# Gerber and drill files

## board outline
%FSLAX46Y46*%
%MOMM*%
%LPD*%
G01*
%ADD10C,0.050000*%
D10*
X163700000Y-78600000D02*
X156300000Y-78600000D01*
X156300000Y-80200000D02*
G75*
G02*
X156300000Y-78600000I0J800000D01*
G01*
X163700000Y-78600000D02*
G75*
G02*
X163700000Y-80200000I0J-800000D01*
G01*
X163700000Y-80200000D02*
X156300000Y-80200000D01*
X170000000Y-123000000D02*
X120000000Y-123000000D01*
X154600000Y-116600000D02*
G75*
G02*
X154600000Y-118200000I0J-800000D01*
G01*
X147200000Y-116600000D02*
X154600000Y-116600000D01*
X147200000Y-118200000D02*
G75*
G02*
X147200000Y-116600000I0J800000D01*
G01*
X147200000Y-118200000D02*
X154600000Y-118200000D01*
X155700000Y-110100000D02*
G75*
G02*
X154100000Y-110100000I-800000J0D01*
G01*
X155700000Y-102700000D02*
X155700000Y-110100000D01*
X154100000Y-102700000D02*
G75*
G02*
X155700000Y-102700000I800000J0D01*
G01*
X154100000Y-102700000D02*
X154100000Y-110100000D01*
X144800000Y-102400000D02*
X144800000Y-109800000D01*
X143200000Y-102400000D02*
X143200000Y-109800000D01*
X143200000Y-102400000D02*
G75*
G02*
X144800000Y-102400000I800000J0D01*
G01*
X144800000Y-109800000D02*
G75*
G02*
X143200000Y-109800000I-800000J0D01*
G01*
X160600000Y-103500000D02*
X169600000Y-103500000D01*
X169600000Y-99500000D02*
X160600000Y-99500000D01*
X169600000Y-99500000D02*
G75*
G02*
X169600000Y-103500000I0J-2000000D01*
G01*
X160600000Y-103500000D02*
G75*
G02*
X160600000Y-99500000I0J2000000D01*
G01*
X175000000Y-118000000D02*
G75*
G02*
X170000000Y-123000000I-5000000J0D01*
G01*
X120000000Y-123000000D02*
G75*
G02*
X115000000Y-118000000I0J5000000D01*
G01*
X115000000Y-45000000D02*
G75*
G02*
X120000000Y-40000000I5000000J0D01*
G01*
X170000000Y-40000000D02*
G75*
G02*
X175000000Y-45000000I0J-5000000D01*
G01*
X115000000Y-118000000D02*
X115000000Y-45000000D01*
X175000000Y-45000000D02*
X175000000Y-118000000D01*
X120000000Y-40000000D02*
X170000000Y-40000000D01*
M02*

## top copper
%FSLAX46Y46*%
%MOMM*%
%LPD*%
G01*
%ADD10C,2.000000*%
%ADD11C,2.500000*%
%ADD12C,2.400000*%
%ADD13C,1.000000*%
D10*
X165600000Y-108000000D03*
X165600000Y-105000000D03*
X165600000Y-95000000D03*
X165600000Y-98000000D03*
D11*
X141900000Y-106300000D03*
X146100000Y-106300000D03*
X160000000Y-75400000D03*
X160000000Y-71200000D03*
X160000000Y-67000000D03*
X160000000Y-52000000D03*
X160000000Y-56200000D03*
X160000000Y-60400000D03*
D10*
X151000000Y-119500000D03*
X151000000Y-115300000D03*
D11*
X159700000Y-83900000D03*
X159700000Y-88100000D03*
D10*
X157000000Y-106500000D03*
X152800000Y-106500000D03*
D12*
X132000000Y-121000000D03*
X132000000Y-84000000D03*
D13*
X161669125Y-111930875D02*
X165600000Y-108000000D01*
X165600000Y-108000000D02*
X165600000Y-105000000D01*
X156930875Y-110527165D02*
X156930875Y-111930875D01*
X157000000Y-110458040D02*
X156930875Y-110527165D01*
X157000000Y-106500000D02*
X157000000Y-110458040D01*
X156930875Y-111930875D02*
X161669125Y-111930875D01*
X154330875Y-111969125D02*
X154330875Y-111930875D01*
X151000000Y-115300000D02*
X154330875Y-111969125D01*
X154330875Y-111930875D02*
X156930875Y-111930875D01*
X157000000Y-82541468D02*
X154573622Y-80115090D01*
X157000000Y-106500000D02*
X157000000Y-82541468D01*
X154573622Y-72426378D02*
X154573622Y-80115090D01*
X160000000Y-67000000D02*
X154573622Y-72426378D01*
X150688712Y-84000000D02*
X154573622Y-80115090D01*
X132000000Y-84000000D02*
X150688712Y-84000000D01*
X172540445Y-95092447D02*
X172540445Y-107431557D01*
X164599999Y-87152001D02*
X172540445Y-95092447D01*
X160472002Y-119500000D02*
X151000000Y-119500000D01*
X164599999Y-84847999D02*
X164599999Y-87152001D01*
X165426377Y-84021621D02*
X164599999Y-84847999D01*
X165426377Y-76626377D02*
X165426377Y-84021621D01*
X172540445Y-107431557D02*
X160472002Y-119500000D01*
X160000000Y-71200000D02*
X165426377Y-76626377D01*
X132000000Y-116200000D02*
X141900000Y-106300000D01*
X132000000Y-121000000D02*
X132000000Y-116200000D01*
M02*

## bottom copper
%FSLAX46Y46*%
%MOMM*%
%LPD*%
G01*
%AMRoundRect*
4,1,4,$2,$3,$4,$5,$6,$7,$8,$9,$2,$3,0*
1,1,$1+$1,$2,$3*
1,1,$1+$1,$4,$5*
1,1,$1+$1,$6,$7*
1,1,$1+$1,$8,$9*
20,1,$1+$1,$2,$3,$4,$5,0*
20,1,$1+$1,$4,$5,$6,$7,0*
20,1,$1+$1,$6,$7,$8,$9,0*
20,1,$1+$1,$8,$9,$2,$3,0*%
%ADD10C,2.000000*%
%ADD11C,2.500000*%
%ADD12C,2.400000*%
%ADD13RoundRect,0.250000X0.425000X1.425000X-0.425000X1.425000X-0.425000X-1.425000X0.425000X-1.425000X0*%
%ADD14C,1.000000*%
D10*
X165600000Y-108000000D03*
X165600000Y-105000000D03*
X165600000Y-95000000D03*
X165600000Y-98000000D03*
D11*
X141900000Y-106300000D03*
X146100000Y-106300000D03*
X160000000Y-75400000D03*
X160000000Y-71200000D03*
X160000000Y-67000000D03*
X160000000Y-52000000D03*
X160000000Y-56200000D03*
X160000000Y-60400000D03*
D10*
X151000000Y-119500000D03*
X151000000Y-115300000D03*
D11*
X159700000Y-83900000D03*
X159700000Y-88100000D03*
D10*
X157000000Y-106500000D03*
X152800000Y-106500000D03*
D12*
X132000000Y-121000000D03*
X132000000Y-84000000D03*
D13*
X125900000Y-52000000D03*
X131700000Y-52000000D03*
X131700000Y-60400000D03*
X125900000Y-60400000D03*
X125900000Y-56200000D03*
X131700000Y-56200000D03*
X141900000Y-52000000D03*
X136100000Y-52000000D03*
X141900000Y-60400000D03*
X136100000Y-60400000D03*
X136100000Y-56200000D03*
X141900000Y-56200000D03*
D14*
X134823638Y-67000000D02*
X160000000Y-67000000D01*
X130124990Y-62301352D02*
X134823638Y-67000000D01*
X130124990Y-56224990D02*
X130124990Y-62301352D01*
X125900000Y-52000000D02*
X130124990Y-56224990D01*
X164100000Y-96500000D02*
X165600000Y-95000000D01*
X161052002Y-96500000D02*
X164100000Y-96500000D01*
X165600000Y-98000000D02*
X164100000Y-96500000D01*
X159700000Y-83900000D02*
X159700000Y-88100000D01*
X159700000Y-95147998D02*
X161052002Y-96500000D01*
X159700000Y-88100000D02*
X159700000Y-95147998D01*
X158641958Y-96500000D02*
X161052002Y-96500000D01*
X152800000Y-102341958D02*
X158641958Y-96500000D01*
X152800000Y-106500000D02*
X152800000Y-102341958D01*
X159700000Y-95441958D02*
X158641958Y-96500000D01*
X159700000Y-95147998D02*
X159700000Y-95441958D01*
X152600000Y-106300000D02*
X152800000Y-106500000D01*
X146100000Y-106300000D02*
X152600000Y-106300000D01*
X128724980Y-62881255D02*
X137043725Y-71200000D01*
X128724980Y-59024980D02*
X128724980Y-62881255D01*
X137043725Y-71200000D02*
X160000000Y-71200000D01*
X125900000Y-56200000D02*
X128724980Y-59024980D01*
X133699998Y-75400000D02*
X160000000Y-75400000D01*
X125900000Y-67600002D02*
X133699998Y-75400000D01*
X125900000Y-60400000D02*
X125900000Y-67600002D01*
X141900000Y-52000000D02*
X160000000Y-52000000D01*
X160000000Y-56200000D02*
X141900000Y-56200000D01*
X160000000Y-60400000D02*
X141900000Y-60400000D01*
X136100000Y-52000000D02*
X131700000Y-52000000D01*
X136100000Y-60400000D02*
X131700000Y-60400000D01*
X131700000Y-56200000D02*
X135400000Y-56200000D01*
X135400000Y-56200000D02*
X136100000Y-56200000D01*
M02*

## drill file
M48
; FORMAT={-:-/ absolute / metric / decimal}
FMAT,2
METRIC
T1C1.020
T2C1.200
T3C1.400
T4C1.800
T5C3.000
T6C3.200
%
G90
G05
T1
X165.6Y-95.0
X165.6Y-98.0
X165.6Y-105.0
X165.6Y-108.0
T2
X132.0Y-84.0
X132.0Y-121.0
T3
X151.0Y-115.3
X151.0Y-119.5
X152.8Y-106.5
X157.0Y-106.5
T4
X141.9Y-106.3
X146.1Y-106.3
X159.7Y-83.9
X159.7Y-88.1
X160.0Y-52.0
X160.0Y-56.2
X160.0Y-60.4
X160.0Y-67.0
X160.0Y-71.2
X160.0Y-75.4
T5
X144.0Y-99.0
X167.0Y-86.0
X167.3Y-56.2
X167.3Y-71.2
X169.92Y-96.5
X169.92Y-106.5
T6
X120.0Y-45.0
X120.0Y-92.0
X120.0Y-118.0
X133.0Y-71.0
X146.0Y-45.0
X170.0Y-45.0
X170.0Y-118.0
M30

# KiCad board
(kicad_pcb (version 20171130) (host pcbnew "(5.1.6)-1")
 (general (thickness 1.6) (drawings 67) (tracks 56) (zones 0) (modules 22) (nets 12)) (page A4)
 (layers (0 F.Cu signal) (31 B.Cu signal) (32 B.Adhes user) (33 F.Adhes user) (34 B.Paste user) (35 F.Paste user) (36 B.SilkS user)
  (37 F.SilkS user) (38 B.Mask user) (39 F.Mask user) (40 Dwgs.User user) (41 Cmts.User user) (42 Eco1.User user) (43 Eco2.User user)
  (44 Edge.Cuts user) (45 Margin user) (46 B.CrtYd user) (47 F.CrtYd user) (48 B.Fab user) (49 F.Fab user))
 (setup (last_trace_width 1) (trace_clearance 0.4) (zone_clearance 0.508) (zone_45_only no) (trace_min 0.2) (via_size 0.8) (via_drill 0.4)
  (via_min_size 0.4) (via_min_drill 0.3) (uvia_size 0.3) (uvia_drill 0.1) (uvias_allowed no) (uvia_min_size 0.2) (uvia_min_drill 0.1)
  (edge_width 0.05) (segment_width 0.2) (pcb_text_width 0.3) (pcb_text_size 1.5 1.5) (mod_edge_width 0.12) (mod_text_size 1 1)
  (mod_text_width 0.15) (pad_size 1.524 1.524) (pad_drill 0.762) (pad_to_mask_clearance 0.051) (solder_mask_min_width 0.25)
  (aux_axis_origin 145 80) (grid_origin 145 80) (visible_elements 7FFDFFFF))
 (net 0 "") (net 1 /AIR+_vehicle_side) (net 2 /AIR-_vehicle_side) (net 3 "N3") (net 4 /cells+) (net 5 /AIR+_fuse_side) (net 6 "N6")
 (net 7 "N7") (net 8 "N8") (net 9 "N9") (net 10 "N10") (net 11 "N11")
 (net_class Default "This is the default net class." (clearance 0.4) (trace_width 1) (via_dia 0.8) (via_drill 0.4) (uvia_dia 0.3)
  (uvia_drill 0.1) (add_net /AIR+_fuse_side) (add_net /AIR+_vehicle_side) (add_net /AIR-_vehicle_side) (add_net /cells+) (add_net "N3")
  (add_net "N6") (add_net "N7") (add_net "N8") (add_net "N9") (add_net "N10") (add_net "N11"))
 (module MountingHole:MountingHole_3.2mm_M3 (layer B.Cu) (at 120 92)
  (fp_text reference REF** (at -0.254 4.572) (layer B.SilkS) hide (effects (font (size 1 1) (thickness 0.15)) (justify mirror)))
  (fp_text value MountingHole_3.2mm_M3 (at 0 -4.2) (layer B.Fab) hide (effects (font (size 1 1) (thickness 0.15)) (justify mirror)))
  (pad 1 np_thru_hole circle (at 0 0) (size 3.2 3.2) (drill 3.2) (layers *.Cu *.Mask)))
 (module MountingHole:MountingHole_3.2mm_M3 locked (layer B.Cu) (at 133 71)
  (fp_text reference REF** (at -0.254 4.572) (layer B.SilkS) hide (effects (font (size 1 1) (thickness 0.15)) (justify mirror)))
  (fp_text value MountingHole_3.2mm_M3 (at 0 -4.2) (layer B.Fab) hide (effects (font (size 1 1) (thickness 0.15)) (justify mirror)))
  (pad 1 np_thru_hole circle (at 0 0) (size 3.2 3.2) (drill 3.2) (layers *.Cu *.Mask)))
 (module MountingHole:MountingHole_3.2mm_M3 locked (layer B.Cu) (at 146 45)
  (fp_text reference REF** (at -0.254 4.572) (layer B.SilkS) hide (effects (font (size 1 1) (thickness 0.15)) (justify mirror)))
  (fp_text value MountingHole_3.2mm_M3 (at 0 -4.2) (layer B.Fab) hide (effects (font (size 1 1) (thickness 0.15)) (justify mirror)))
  (pad 1 np_thru_hole circle (at 0 0) (size 3.2 3.2) (drill 3.2) (layers *.Cu *.Mask)))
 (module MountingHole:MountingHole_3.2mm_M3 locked (layer B.Cu) (at 170 45 180)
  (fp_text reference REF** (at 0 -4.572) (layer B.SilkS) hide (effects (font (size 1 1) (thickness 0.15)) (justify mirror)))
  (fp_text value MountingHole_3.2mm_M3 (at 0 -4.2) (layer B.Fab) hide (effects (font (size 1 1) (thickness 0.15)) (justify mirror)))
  (pad 1 np_thru_hole circle (at 0 0 180) (size 3.2 3.2) (drill 3.2) (layers *.Cu *.Mask)))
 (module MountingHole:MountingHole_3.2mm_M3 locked (layer B.Cu) (at 120 118)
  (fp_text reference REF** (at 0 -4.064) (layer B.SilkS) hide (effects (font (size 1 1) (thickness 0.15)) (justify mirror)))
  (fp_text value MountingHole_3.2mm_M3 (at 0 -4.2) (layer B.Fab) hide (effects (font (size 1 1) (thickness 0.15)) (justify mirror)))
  (pad 1 np_thru_hole circle (at 0 0) (size 3.2 3.2) (drill 3.2) (layers *.Cu *.Mask)))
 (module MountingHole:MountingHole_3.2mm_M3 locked (layer B.Cu) (at 170 118 180)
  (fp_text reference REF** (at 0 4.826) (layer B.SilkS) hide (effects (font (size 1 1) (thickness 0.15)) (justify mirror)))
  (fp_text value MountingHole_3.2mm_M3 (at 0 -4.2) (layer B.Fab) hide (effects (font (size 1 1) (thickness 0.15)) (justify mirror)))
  (pad 1 np_thru_hole circle (at 0 0 180) (size 3.2 3.2) (drill 3.2) (layers *.Cu *.Mask)))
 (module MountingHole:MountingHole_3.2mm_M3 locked (layer B.Cu) (at 120 45)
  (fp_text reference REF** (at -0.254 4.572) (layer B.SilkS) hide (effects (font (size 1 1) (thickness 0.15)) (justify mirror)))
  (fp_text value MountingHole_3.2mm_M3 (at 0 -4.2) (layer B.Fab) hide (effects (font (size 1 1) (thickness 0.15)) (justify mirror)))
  (pad 1 np_thru_hole circle (at 0 0) (size 3.2 3.2) (drill 3.2) (layers *.Cu *.Mask)))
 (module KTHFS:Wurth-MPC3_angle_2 (layer F.Cu) (at 165.6 105 90)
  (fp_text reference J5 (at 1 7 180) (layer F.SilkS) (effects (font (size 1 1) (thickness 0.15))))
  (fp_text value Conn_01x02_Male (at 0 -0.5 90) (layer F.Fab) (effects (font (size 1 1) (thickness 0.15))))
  (pad "" np_thru_hole circle (at -1.5 4.32 90) (size 3 3) (drill 3) (layers *.Cu *.Mask))
  (pad 2 thru_hole circle (at -3 0 90) (size 2 2) (drill 1.02) (layers *.Cu *.Mask) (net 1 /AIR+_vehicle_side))
  (pad 1 thru_hole circle (at 0 0 90) (size 2 2) (drill 1.02) (layers *.Cu *.Mask) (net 1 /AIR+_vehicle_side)))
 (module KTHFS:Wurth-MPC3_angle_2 (layer F.Cu) (at 165.6 95 90)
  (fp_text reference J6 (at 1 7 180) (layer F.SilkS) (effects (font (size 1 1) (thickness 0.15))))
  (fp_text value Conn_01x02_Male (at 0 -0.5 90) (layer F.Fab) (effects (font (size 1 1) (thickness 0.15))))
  (pad 1 thru_hole circle (at 0 0 90) (size 2 2) (drill 1.02) (layers *.Cu *.Mask) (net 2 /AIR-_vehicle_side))
  (pad 2 thru_hole circle (at -3 0 90) (size 2 2) (drill 1.02) (layers *.Cu *.Mask) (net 2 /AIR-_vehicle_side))
  (pad "" np_thru_hole circle (at -1.5 4.32 90) (size 3 3) (drill 3) (layers *.Cu *.Mask)))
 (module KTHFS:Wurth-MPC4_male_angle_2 (layer F.Cu) (at 144 99 180)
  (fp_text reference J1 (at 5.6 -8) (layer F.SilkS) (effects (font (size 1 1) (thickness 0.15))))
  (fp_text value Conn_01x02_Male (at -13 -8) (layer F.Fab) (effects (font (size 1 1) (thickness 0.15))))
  (pad "" np_thru_hole circle (at 0 0 180) (size 3 3) (drill 3) (layers *.Cu *.Mask))
  (pad 1 thru_hole circle (at 2.1 -7.3 180) (size 2.5 2.5) (drill 1.8) (layers *.Cu *.Mask) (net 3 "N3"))
  (pad 2 thru_hole circle (at -2.1 -7.3 180) (size 2.5 2.5) (drill 1.8) (layers *.Cu *.Mask) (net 2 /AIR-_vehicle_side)))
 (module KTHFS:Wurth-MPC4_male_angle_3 (layer F.Cu) (at 160 67 90)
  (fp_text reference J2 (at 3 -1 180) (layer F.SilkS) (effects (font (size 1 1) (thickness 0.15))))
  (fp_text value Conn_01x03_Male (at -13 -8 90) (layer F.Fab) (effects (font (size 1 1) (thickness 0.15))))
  (pad 3 thru_hole circle (at -8.4 0 90) (size 2.5 2.5) (drill 1.8) (layers *.Cu *.Mask) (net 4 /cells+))
  (pad 2 thru_hole circle (at -4.2 0 90) (size 2.5 2.5) (drill 1.8) (layers *.Cu *.Mask) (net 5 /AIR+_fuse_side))
  (pad 1 thru_hole circle (at 0 0 90) (size 2.5 2.5) (drill 1.8) (layers *.Cu *.Mask) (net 1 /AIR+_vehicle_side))
  (pad "" np_thru_hole circle (at -4.2 7.3 90) (size 3 3) (drill 3) (layers *.Cu *.Mask)))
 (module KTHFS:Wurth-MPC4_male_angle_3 (layer F.Cu) (at 160 52 90)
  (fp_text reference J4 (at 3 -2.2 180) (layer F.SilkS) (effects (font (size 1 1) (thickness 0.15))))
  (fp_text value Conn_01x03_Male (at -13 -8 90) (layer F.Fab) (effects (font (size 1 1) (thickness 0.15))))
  (pad "" np_thru_hole circle (at -4.2 7.3 90) (size 3 3) (drill 3) (layers *.Cu *.Mask))
  (pad 1 thru_hole circle (at 0 0 90) (size 2.5 2.5) (drill 1.8) (layers *.Cu *.Mask) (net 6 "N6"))
  (pad 2 thru_hole circle (at -4.2 0 90) (size 2.5 2.5) (drill 1.8) (layers *.Cu *.Mask) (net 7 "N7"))
  (pad 3 thru_hole circle (at -8.4 0 90) (size 2.5 2.5) (drill 1.8) (layers *.Cu *.Mask) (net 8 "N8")))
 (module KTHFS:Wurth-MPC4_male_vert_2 (layer F.Cu) (at 151 119.5 90)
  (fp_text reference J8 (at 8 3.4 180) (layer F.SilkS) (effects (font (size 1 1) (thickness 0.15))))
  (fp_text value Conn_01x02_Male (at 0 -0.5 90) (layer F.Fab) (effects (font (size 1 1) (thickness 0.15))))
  (pad 1 thru_hole circle (at 0 0 90) (size 2 2) (drill 1.4) (layers *.Cu *.Mask) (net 5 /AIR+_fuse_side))
  (pad 2 thru_hole circle (at 4.2 0 90) (size 2 2) (drill 1.4) (layers *.Cu *.Mask) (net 1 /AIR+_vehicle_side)))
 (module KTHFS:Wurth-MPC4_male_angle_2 (layer F.Cu) (at 167 86 90)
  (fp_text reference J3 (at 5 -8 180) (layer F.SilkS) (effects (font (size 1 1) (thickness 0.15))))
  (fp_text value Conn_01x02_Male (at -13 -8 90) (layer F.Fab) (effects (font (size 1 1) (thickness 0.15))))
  (pad "" np_thru_hole circle (at 0 0 90) (size 3 3) (drill 3) (layers *.Cu *.Mask))
  (pad 1 thru_hole circle (at 2.1 -7.3 90) (size 2.5 2.5) (drill 1.8) (layers *.Cu *.Mask) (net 2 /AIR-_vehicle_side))
  (pad 2 thru_hole circle (at -2.1 -7.3 90) (size 2.5 2.5) (drill 1.8) (layers *.Cu *.Mask) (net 2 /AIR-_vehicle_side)))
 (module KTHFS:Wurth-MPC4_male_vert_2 (layer F.Cu) (at 157 106.5 180)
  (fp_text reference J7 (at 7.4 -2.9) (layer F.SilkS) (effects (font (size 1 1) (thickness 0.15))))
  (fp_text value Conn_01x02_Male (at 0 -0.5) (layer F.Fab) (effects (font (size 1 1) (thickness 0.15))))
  (pad 1 thru_hole circle (at 0 0 180) (size 2 2) (drill 1.4) (layers *.Cu *.Mask) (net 1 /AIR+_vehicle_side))
  (pad 2 thru_hole circle (at 4.2 0 180) (size 2 2) (drill 1.4) (layers *.Cu *.Mask) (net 2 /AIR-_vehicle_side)))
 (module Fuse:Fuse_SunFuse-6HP (layer F.Cu) (at 132 121 90)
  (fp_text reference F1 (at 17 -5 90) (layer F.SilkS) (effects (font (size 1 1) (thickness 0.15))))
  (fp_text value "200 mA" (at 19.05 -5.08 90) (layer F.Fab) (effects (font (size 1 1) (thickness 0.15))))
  (pad 1 thru_hole circle (at 0 0 90) (size 2.4 2.4) (drill 1.2) (layers *.Cu *.Mask) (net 3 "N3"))
  (pad 2 thru_hole circle (at 37 0 90) (size 2.4 2.4) (drill 1.2) (layers *.Cu *.Mask) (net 1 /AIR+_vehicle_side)))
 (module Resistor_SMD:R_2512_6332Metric (layer B.Cu) (at 128.8 52 180)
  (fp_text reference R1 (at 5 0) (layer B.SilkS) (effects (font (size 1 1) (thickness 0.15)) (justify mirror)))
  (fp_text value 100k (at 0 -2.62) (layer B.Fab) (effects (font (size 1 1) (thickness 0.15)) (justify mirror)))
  (pad 2 smd roundrect (at 2.9 0 180) (size 1.35 3.35) (layers B.Cu B.Paste B.Mask) (roundrect_rratio 0.185185) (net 1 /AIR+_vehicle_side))
  (pad 1 smd roundrect (at -2.9 0 180) (size 1.35 3.35) (layers B.Cu B.Paste B.Mask) (roundrect_rratio 0.185185) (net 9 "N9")))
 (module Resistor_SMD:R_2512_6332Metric (layer B.Cu) (at 128.8 60.4 180)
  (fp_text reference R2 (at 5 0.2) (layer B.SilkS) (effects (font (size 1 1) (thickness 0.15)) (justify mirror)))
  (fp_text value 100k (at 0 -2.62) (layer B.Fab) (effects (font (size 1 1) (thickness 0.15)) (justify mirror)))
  (pad 1 smd roundrect (at -2.9 0 180) (size 1.35 3.35) (layers B.Cu B.Paste B.Mask) (roundrect_rratio 0.185185) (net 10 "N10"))
  (pad 2 smd roundrect (at 2.9 0 180) (size 1.35 3.35) (layers B.Cu B.Paste B.Mask) (roundrect_rratio 0.185185) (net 4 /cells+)))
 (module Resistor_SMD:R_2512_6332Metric (layer B.Cu) (at 128.8 56.2 180)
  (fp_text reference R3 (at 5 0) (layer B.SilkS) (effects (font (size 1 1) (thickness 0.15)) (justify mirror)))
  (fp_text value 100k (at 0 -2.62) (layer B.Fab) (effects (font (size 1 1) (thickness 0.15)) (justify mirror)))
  (pad 2 smd roundrect (at 2.9 0 180) (size 1.35 3.35) (layers B.Cu B.Paste B.Mask) (roundrect_rratio 0.185185) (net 5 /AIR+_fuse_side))
  (pad 1 smd roundrect (at -2.9 0 180) (size 1.35 3.35) (layers B.Cu B.Paste B.Mask) (roundrect_rratio 0.185185) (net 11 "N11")))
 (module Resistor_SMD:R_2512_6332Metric (layer B.Cu) (at 139 52 180)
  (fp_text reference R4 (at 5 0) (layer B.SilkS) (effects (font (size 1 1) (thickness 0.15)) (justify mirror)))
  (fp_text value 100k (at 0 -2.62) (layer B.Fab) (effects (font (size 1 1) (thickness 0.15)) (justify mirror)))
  (pad 1 smd roundrect (at -2.9 0 180) (size 1.35 3.35) (layers B.Cu B.Paste B.Mask) (roundrect_rratio 0.185185) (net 6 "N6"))
  (pad 2 smd roundrect (at 2.9 0 180) (size 1.35 3.35) (layers B.Cu B.Paste B.Mask) (roundrect_rratio 0.185185) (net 9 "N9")))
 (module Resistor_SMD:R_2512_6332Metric (layer B.Cu) (at 139 60.4 180)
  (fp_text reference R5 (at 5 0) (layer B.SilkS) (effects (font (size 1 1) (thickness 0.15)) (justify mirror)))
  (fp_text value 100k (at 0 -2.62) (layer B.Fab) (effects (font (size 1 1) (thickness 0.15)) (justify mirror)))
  (pad 1 smd roundrect (at -2.9 0 180) (size 1.35 3.35) (layers B.Cu B.Paste B.Mask) (roundrect_rratio 0.185185) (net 8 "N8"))
  (pad 2 smd roundrect (at 2.9 0 180) (size 1.35 3.35) (layers B.Cu B.Paste B.Mask) (roundrect_rratio 0.185185) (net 10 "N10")))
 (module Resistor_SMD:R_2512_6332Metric (layer B.Cu) (at 139 56.2 180)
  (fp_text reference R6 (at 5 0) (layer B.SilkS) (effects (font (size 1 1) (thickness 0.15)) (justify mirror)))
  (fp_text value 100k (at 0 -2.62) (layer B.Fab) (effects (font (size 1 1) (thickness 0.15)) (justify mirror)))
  (pad 2 smd roundrect (at 2.9 0 180) (size 1.35 3.35) (layers B.Cu B.Paste B.Mask) (roundrect_rratio 0.185185) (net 11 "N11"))
  (pad 1 smd roundrect (at -2.9 0 180) (size 1.35 3.35) (layers B.Cu B.Paste B.Mask) (roundrect_rratio 0.185185) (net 7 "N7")))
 (gr_line (start 163.7 78.6) (end 156.3 78.6) (layer Edge.Cuts) (width 0.05))
 (gr_arc (start 156.3 79.4) (end 156.3 78.6) (angle -180) (layer Edge.Cuts) (width 0.05))
 (gr_arc (start 163.7 79.4) (end 163.7 80.2) (angle -180) (layer Edge.Cuts) (width 0.05))
 (gr_line (start 163.7 80.2) (end 156.3 80.2) (layer Edge.Cuts) (width 0.05))
 (gr_line (start 170 123) (end 120 123) (layer Edge.Cuts) (width 0.05))
 (gr_arc (start 154.6 117.4) (end 154.6 118.2) (angle -180) (layer Edge.Cuts) (width 0.05))
 (gr_line (start 147.2 116.6) (end 154.6 116.6) (layer Edge.Cuts) (width 0.05))
 (gr_arc (start 147.2 117.4) (end 147.2 116.6) (angle -180) (layer Edge.Cuts) (width 0.05))
 (gr_line (start 147.2 118.2) (end 154.6 118.2) (layer Edge.Cuts) (width 0.05))
 (gr_arc (start 154.9 110.1) (end 154.1 110.1) (angle -180) (layer Edge.Cuts) (width 0.05))
 (gr_line (start 155.7 102.7) (end 155.7 110.1) (layer Edge.Cuts) (width 0.05))
 (gr_arc (start 154.9 102.7) (end 155.7 102.7) (angle -180) (layer Edge.Cuts) (width 0.05))
 (gr_line (start 154.1 102.7) (end 154.1 110.1) (layer Edge.Cuts) (width 0.05))
 (gr_line (start 144.8 102.4) (end 144.8 109.8) (layer Edge.Cuts) (width 0.05))
 (gr_line (start 143.2 102.4) (end 143.2 109.8) (layer Edge.Cuts) (width 0.05))
 (gr_arc (start 144 102.4) (end 144.8 102.4) (angle -180) (layer Edge.Cuts) (width 0.05))
 (gr_arc (start 144 109.8) (end 143.2 109.8) (angle -180) (layer Edge.Cuts) (width 0.05))
 (gr_line (start 160.6 103.5) (end 169.6 103.5) (layer Edge.Cuts) (width 0.05))
 (gr_line (start 169.6 99.5) (end 160.6 99.5) (layer Edge.Cuts) (width 0.05))
 (gr_arc (start 169.6 101.5) (end 169.6 103.5) (angle -180) (layer Edge.Cuts) (width 0.05))
 (gr_arc (start 160.6 101.5) (end 160.6 99.5) (angle -180) (layer Edge.Cuts) (width 0.05))
 (gr_arc (start 170 118) (end 170 123) (angle -90) (layer Edge.Cuts) (width 0.05))
 (gr_arc (start 120 118) (end 115 118) (angle -90) (layer Edge.Cuts) (width 0.05))
 (gr_arc (start 120 45) (end 120 40) (angle -90) (layer Edge.Cuts) (width 0.05))
 (gr_arc (start 170 45) (end 175 45) (angle -90) (layer Edge.Cuts) (width 0.05))
 (gr_line (start 115 118) (end 115 45) (layer Edge.Cuts) (width 0.05))
 (gr_line (start 175 45) (end 175 118) (layer Edge.Cuts) (width 0.05))
 (gr_line (start 120 40) (end 170 40) (layer Edge.Cuts) (width 0.05))
 (segment (start 161.669125 111.930875) (end 165.6 108) (width 1) (layer F.Cu) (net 1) (status 20))
 (segment (start 165.6 108) (end 165.6 105) (width 1) (layer F.Cu) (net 1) (status 30))
 (segment (start 156.930875 110.527165) (end 156.930875 111.930875) (width 1) (layer F.Cu) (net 1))
 (segment (start 157 110.45804) (end 156.930875 110.527165) (width 1) (layer F.Cu) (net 1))
 (segment (start 157 106.5) (end 157 110.45804) (width 1) (layer F.Cu) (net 1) (status 10))
 (segment (start 156.930875 111.930875) (end 161.669125 111.930875) (width 1) (layer F.Cu) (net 1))
 (segment (start 154.330875 111.969125) (end 154.330875 111.930875) (width 1) (layer F.Cu) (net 1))
 (segment (start 151 115.3) (end 154.330875 111.969125) (width 1) (layer F.Cu) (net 1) (status 10))
 (segment (start 154.330875 111.930875) (end 156.930875 111.930875) (width 1) (layer F.Cu) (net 1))
 (segment (start 157 82.541468) (end 154.573622 80.11509) (width 1) (layer F.Cu) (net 1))
 (segment (start 157 106.5) (end 157 82.541468) (width 1) (layer F.Cu) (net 1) (status 10))
 (segment (start 154.573622 72.426378) (end 154.573622 80.11509) (width 1) (layer F.Cu) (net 1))
 (segment (start 160 67) (end 154.573622 72.426378) (width 1) (layer F.Cu) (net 1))
 (segment (start 134.823638 67) (end 160 67) (width 1) (layer B.Cu) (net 1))
 (segment (start 130.12499 62.301352) (end 134.823638 67) (width 1) (layer B.Cu) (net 1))
 (segment (start 130.12499 56.22499) (end 130.12499 62.301352) (width 1) (layer B.Cu) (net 1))
 (segment (start 125.9 52) (end 130.12499 56.22499) (width 1) (layer B.Cu) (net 1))
 (segment (start 150.688712 84) (end 154.573622 80.11509) (width 1) (layer F.Cu) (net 1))
 (segment (start 132 84) (end 150.688712 84) (width 1) (layer F.Cu) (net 1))
 (segment (start 164.1 96.5) (end 165.6 95) (width 1) (layer B.Cu) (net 2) (status 20))
 (segment (start 161.052002 96.5) (end 164.1 96.5) (width 1) (layer B.Cu) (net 2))
 (segment (start 165.6 98) (end 164.1 96.5) (width 1) (layer B.Cu) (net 2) (status 10))
 (segment (start 159.7 83.9) (end 159.7 88.1) (width 1) (layer B.Cu) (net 2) (status 30))
 (segment (start 159.7 95.147998) (end 161.052002 96.5) (width 1) (layer B.Cu) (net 2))
 (segment (start 159.7 88.1) (end 159.7 95.147998) (width 1) (layer B.Cu) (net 2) (status 10))
 (segment (start 158.641958 96.5) (end 161.052002 96.5) (width 1) (layer B.Cu) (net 2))
 (segment (start 152.8 102.341958) (end 158.641958 96.5) (width 1) (layer B.Cu) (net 2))
 (segment (start 152.8 106.5) (end 152.8 102.341958) (width 1) (layer B.Cu) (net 2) (status 10))
 (segment (start 159.7 95.441958) (end 158.641958 96.5) (width 1) (layer B.Cu) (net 2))
 (segment (start 159.7 95.147998) (end 159.7 95.441958) (width 1) (layer B.Cu) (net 2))
 (segment (start 152.6 106.3) (end 152.8 106.5) (width 1) (layer B.Cu) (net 2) (status 30))
 (segment (start 146.1 106.3) (end 152.6 106.3) (width 1) (layer B.Cu) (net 2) (status 30))
 (segment (start 172.540445 95.092447) (end 172.540445 107.431557) (width 1) (layer F.Cu) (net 5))
 (segment (start 164.599999 87.152001) (end 172.540445 95.092447) (width 1) (layer F.Cu) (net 5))
 (segment (start 160.472002 119.5) (end 151 119.5) (width 1) (layer F.Cu) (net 5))
 (segment (start 164.599999 84.847999) (end 164.599999 87.152001) (width 1) (layer F.Cu) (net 5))
 (segment (start 165.426377 84.021621) (end 164.599999 84.847999) (width 1) (layer F.Cu) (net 5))
 (segment (start 165.426377 76.626377) (end 165.426377 84.021621) (width 1) (layer F.Cu) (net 5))
 (segment (start 172.540445 107.431557) (end 160.472002 119.5) (width 1) (layer F.Cu) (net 5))
 (segment (start 160 71.2) (end 165.426377 76.626377) (width 1) (layer F.Cu) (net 5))
 (segment (start 128.72498 62.881255) (end 137.043725 71.2) (width 1) (layer B.Cu) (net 5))
 (segment (start 128.72498 59.02498) (end 128.72498 62.881255) (width 1) (layer B.Cu) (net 5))
 (segment (start 137.043725 71.2) (end 160 71.2) (width 1) (layer B.Cu) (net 5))
 (segment (start 125.9 56.2) (end 128.72498 59.02498) (width 1) (layer B.Cu) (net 5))
 (segment (start 133.699998 75.4) (end 160 75.4) (width 1) (layer B.Cu) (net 4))
 (segment (start 125.9 67.600002) (end 133.699998 75.4) (width 1) (layer B.Cu) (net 4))
 (segment (start 125.9 60.4) (end 125.9 67.600002) (width 1) (layer B.Cu) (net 4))
 (segment (start 132 116.2) (end 141.9 106.3) (width 1) (layer F.Cu) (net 3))
 (segment (start 132 121) (end 132 116.2) (width 1) (layer F.Cu) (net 3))
 (segment (start 141.9 52) (end 160 52) (width 1) (layer B.Cu) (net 6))
 (segment (start 160 56.2) (end 141.9 56.2) (width 1) (layer B.Cu) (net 7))
 (segment (start 160 60.4) (end 141.9 60.4) (width 1) (layer B.Cu) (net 8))
 (segment (start 136.1 52) (end 131.7 52) (width 1) (layer B.Cu) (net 9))
 (segment (start 136.1 60.4) (end 131.7 60.4) (width 1) (layer B.Cu) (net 10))
 (segment (start 131.7 56.2) (end 135.4 56.2) (width 1) (layer B.Cu) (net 11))
 (segment (start 135.4 56.2) (end 136.1 56.2) (width 1) (layer B.Cu) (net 11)))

